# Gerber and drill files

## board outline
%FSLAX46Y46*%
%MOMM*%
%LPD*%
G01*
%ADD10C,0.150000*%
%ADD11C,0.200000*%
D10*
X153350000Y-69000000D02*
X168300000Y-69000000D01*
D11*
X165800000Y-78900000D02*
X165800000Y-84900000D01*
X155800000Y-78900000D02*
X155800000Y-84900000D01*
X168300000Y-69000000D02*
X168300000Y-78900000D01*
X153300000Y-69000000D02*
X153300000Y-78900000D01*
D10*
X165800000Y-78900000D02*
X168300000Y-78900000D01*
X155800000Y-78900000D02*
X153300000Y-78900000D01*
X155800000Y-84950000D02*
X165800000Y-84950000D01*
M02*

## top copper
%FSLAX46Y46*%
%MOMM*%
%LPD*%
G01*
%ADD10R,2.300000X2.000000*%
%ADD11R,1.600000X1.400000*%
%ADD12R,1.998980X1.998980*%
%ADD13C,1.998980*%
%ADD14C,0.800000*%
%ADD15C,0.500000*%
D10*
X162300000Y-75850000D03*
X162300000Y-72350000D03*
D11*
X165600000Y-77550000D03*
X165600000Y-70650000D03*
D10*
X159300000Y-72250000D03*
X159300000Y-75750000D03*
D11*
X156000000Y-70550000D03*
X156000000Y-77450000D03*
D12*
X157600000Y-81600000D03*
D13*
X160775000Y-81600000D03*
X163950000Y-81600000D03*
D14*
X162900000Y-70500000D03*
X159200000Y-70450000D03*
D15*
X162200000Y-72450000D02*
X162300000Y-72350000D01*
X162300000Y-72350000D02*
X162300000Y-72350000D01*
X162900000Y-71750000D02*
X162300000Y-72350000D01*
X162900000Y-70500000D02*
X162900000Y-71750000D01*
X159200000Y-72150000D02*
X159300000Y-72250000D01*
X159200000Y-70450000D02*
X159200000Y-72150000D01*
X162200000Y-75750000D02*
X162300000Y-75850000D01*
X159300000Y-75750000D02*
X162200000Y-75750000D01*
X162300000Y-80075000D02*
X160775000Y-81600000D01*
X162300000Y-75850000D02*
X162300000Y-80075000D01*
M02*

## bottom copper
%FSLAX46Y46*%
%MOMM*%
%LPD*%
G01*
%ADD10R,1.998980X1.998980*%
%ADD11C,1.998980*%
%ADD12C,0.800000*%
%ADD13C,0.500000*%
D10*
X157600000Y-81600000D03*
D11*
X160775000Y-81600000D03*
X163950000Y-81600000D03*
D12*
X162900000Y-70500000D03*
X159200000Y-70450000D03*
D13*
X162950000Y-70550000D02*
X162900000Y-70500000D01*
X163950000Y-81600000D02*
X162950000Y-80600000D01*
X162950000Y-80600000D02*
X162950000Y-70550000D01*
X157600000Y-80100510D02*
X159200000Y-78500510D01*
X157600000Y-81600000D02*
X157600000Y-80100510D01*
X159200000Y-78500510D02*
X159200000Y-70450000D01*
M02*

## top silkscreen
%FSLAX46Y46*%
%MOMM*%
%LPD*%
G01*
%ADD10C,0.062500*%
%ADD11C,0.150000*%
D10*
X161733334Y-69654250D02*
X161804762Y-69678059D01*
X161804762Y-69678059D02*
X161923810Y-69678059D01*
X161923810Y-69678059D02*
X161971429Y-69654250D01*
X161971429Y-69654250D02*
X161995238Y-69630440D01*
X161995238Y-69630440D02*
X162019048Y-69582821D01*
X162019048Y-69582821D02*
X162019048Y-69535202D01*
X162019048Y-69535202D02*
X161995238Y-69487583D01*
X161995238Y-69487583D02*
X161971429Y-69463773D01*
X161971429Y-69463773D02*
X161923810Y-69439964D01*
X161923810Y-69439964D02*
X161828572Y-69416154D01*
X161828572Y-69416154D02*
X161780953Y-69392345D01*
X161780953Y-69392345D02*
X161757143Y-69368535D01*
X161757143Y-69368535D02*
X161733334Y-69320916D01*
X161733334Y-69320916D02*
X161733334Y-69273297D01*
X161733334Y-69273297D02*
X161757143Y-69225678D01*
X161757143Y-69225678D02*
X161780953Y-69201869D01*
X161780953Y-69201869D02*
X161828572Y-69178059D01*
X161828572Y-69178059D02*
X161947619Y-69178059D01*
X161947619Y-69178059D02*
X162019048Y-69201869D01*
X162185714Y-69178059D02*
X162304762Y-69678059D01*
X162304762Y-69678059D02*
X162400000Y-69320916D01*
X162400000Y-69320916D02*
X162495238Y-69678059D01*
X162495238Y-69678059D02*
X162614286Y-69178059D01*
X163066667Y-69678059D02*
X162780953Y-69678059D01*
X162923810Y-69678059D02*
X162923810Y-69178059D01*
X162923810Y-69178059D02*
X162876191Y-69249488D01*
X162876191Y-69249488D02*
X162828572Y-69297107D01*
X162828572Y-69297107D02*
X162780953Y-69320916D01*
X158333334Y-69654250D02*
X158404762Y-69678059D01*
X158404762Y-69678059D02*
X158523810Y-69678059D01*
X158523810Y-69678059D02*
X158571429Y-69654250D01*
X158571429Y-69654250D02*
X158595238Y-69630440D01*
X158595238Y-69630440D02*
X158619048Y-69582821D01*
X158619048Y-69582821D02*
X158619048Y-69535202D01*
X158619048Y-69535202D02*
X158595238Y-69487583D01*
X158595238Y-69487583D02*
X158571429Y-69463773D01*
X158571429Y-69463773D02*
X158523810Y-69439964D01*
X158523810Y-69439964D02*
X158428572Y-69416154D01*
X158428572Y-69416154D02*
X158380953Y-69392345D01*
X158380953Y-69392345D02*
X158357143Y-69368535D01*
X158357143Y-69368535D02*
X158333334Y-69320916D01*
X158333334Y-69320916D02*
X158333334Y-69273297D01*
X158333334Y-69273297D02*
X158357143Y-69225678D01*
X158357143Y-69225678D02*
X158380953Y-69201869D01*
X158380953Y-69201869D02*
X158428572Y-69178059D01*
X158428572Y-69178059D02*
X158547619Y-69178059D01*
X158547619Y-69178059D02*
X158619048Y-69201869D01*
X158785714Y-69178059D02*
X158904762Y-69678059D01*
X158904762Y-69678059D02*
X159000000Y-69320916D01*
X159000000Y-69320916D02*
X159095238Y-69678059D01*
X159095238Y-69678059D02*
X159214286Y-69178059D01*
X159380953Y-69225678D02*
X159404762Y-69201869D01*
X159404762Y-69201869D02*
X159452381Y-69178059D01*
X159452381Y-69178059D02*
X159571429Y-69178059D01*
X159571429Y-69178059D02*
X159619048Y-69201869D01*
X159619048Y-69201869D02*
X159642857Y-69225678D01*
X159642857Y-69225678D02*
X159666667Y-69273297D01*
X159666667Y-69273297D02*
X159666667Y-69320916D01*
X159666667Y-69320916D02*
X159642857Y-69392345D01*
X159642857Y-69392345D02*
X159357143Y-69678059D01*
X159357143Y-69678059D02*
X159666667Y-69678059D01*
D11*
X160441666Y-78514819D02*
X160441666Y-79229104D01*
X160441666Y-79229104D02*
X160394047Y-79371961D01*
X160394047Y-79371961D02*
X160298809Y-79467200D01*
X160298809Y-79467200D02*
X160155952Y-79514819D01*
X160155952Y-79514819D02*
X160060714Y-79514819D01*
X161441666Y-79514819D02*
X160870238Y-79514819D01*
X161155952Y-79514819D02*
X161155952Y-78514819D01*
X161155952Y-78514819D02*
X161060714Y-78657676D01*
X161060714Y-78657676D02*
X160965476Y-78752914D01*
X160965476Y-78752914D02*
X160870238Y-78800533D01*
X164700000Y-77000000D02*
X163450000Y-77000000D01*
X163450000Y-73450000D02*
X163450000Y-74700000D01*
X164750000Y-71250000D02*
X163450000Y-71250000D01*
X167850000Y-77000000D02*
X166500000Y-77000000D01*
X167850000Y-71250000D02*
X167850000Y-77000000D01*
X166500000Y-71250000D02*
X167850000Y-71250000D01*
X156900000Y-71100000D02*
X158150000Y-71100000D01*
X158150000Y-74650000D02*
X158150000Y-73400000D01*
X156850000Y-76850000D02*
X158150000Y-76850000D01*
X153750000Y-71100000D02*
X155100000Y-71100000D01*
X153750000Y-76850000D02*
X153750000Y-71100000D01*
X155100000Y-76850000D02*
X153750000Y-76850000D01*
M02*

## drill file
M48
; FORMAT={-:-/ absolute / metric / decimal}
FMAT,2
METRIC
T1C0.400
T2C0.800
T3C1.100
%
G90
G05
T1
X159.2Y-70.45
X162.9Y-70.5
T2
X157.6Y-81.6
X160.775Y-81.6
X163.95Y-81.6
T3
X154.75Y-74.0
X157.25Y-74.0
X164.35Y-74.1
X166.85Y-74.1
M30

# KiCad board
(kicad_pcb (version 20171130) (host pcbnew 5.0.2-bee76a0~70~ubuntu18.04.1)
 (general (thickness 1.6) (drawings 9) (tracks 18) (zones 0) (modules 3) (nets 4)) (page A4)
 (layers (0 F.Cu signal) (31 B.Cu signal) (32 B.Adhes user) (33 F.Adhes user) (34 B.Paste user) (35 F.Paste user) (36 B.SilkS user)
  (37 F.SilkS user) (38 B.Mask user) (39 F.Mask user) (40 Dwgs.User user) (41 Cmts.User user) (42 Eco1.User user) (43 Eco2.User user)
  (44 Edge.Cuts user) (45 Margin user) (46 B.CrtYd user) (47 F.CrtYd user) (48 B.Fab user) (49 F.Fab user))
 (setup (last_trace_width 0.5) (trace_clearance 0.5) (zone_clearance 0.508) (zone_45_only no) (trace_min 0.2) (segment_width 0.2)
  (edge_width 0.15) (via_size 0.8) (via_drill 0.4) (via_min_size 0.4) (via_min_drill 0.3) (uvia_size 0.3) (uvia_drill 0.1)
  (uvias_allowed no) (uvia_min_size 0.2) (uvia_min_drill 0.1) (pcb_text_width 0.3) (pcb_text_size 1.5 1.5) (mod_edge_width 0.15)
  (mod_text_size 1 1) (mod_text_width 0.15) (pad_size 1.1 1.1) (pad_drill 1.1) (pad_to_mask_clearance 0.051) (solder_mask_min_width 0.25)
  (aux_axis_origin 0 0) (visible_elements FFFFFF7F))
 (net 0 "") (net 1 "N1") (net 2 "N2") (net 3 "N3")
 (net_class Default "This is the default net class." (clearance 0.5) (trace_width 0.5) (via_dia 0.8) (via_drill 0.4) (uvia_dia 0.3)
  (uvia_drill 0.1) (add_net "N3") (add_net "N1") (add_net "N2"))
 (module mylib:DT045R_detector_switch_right (layer F.Cu) (at 165.6 74.1 270)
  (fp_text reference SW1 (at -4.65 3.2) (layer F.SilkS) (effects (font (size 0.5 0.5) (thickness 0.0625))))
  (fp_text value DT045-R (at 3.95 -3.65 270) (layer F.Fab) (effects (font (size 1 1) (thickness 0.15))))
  (fp_line (start 2.9 0.9) (end 2.9 2.15) (layer F.SilkS) (width 0.15))
  (fp_line (start -0.65 2.15) (end 0.6 2.15) (layer F.SilkS) (width 0.15))
  (fp_line (start -2.85 0.85) (end -2.85 2.15) (layer F.SilkS) (width 0.15))
  (fp_line (start 2.9 -2.25) (end 2.9 -0.9) (layer F.SilkS) (width 0.15))
  (fp_line (start -2.85 -2.25) (end 2.9 -2.25) (layer F.SilkS) (width 0.15))
  (fp_line (start -2.85 -0.9) (end -2.85 -2.25) (layer F.SilkS) (width 0.15))
  (pad 1 smd rect (at 1.75 3.3 270) (size 2 2.3) (layers F.Cu F.Paste F.Mask) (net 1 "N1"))
  (pad 2 smd rect (at -1.75 3.3 270) (size 2 2.3) (layers F.Cu F.Paste F.Mask) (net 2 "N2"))
  (pad "" np_thru_hole circle (at 0 1.25 270) (size 1.1 1.1) (drill 1.1) (layers *.Cu *.Mask))
  (pad "" np_thru_hole circle (at 0 -1.25 270) (size 1.1 1.1) (drill 1.1) (layers *.Cu *.Mask))
  (pad 3 smd rect (at 3.45 0 270) (size 1.4 1.6) (layers F.Cu F.Paste F.Mask))
  (pad 3 smd rect (at -3.45 0 270) (size 1.4 1.6) (layers F.Cu F.Paste F.Mask)))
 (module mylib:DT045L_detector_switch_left (layer F.Cu) (at 156 74 90)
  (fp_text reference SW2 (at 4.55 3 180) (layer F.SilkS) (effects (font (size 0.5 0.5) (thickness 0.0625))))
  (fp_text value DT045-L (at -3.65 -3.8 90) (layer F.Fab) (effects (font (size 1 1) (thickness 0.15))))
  (fp_line (start 2.9 0.9) (end 2.9 2.15) (layer F.SilkS) (width 0.15))
  (fp_line (start -0.65 2.15) (end 0.6 2.15) (layer F.SilkS) (width 0.15))
  (fp_line (start -2.85 0.85) (end -2.85 2.15) (layer F.SilkS) (width 0.15))
  (fp_line (start 2.9 -2.25) (end 2.9 -0.9) (layer F.SilkS) (width 0.15))
  (fp_line (start -2.85 -2.25) (end 2.9 -2.25) (layer F.SilkS) (width 0.15))
  (fp_line (start -2.85 -0.9) (end -2.85 -2.25) (layer F.SilkS) (width 0.15))
  (pad 1 smd rect (at 1.75 3.3 90) (size 2 2.3) (layers F.Cu F.Paste F.Mask) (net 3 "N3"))
  (pad 2 smd rect (at -1.75 3.3 90) (size 2 2.3) (layers F.Cu F.Paste F.Mask) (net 1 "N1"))
  (pad "" np_thru_hole circle (at 0 1.25 90) (size 1.1 1.1) (drill 1.1) (layers *.Cu *.Mask))
  (pad "" np_thru_hole circle (at 0 -1.25 90) (size 1.1 1.1) (drill 1.1) (layers *.Cu *.Mask))
  (pad 3 smd rect (at 3.45 0 90) (size 1.4 1.6) (layers F.Cu F.Paste F.Mask))
  (pad 3 smd rect (at -3.45 0 90) (size 1.4 1.6) (layers F.Cu F.Paste F.Mask)))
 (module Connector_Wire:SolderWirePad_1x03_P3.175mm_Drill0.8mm (layer F.Cu) (at 157.6 81.6)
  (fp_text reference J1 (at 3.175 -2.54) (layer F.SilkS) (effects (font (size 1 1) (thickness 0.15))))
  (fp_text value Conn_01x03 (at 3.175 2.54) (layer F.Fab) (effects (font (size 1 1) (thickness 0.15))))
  (pad 1 thru_hole rect (at 0 0) (size 1.99898 1.99898) (drill 0.8001) (layers *.Cu *.Mask) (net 3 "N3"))
  (pad 2 thru_hole circle (at 3.175 0) (size 1.99898 1.99898) (drill 0.8001) (layers *.Cu *.Mask) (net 1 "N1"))
  (pad 3 thru_hole circle (at 6.35 0) (size 1.99898 1.99898) (drill 0.8001) (layers *.Cu *.Mask) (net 2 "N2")))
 (gr_line (start 153.35 69) (end 168.3 69) (layer Edge.Cuts) (width 0.15))
 (gr_line (start 165.8 78.9) (end 165.8 84.9) (layer Edge.Cuts) (width 0.2))
 (gr_line (start 155.8 78.9) (end 155.8 84.9) (layer Edge.Cuts) (width 0.2))
 (gr_line (start 168.3 69) (end 168.3 78.9) (layer Edge.Cuts) (width 0.2))
 (gr_line (start 153.3 69) (end 153.3 78.9) (layer Edge.Cuts) (width 0.2))
 (gr_line (start 165.8 78.9) (end 168.3 78.9) (layer Edge.Cuts) (width 0.15))
 (gr_line (start 155.8 78.9) (end 153.3 78.9) (layer Edge.Cuts) (width 0.15))
 (gr_line (start 155.8 84.95) (end 165.8 84.95) (layer Edge.Cuts) (width 0.15))
 (segment (start 162.2 72.45) (end 162.3 72.35) (width 0.5) (layer F.Cu) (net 2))
 (segment (start 162.3 72.35) (end 162.3 72.35) (width 0.5) (layer F.Cu) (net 2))
 (via (at 162.9 70.5) (size 0.8) (drill 0.4) (layers F.Cu B.Cu) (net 2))
 (segment (start 162.95 70.55) (end 162.9 70.5) (width 0.5) (layer B.Cu) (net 2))
 (segment (start 163.95 81.6) (end 162.95 80.6) (width 0.5) (layer B.Cu) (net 2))
 (segment (start 162.95 80.6) (end 162.95 70.55) (width 0.5) (layer B.Cu) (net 2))
 (segment (start 162.9 71.75) (end 162.3 72.35) (width 0.5) (layer F.Cu) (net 2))
 (segment (start 162.9 70.5) (end 162.9 71.75) (width 0.5) (layer F.Cu) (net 2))
 (segment (start 157.6 80.10051) (end 159.2 78.50051) (width 0.5) (layer B.Cu) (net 3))
 (segment (start 157.6 81.6) (end 157.6 80.10051) (width 0.5) (layer B.Cu) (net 3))
 (via (at 159.2 70.45) (size 0.8) (drill 0.4) (layers F.Cu B.Cu) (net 3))
 (segment (start 159.2 78.50051) (end 159.2 70.45) (width 0.5) (layer B.Cu) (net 3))
 (segment (start 159.2 72.15) (end 159.3 72.25) (width 0.5) (layer F.Cu) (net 3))
 (segment (start 159.2 70.45) (end 159.2 72.15) (width 0.5) (layer F.Cu) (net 3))
 (segment (start 162.2 75.75) (end 162.3 75.85) (width 0.5) (layer F.Cu) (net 1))
 (segment (start 159.3 75.75) (end 162.2 75.75) (width 0.5) (layer F.Cu) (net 1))
 (segment (start 162.3 80.075) (end 160.775 81.6) (width 0.5) (layer F.Cu) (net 1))
 (segment (start 162.3 75.85) (end 162.3 80.075) (width 0.5) (layer F.Cu) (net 1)))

